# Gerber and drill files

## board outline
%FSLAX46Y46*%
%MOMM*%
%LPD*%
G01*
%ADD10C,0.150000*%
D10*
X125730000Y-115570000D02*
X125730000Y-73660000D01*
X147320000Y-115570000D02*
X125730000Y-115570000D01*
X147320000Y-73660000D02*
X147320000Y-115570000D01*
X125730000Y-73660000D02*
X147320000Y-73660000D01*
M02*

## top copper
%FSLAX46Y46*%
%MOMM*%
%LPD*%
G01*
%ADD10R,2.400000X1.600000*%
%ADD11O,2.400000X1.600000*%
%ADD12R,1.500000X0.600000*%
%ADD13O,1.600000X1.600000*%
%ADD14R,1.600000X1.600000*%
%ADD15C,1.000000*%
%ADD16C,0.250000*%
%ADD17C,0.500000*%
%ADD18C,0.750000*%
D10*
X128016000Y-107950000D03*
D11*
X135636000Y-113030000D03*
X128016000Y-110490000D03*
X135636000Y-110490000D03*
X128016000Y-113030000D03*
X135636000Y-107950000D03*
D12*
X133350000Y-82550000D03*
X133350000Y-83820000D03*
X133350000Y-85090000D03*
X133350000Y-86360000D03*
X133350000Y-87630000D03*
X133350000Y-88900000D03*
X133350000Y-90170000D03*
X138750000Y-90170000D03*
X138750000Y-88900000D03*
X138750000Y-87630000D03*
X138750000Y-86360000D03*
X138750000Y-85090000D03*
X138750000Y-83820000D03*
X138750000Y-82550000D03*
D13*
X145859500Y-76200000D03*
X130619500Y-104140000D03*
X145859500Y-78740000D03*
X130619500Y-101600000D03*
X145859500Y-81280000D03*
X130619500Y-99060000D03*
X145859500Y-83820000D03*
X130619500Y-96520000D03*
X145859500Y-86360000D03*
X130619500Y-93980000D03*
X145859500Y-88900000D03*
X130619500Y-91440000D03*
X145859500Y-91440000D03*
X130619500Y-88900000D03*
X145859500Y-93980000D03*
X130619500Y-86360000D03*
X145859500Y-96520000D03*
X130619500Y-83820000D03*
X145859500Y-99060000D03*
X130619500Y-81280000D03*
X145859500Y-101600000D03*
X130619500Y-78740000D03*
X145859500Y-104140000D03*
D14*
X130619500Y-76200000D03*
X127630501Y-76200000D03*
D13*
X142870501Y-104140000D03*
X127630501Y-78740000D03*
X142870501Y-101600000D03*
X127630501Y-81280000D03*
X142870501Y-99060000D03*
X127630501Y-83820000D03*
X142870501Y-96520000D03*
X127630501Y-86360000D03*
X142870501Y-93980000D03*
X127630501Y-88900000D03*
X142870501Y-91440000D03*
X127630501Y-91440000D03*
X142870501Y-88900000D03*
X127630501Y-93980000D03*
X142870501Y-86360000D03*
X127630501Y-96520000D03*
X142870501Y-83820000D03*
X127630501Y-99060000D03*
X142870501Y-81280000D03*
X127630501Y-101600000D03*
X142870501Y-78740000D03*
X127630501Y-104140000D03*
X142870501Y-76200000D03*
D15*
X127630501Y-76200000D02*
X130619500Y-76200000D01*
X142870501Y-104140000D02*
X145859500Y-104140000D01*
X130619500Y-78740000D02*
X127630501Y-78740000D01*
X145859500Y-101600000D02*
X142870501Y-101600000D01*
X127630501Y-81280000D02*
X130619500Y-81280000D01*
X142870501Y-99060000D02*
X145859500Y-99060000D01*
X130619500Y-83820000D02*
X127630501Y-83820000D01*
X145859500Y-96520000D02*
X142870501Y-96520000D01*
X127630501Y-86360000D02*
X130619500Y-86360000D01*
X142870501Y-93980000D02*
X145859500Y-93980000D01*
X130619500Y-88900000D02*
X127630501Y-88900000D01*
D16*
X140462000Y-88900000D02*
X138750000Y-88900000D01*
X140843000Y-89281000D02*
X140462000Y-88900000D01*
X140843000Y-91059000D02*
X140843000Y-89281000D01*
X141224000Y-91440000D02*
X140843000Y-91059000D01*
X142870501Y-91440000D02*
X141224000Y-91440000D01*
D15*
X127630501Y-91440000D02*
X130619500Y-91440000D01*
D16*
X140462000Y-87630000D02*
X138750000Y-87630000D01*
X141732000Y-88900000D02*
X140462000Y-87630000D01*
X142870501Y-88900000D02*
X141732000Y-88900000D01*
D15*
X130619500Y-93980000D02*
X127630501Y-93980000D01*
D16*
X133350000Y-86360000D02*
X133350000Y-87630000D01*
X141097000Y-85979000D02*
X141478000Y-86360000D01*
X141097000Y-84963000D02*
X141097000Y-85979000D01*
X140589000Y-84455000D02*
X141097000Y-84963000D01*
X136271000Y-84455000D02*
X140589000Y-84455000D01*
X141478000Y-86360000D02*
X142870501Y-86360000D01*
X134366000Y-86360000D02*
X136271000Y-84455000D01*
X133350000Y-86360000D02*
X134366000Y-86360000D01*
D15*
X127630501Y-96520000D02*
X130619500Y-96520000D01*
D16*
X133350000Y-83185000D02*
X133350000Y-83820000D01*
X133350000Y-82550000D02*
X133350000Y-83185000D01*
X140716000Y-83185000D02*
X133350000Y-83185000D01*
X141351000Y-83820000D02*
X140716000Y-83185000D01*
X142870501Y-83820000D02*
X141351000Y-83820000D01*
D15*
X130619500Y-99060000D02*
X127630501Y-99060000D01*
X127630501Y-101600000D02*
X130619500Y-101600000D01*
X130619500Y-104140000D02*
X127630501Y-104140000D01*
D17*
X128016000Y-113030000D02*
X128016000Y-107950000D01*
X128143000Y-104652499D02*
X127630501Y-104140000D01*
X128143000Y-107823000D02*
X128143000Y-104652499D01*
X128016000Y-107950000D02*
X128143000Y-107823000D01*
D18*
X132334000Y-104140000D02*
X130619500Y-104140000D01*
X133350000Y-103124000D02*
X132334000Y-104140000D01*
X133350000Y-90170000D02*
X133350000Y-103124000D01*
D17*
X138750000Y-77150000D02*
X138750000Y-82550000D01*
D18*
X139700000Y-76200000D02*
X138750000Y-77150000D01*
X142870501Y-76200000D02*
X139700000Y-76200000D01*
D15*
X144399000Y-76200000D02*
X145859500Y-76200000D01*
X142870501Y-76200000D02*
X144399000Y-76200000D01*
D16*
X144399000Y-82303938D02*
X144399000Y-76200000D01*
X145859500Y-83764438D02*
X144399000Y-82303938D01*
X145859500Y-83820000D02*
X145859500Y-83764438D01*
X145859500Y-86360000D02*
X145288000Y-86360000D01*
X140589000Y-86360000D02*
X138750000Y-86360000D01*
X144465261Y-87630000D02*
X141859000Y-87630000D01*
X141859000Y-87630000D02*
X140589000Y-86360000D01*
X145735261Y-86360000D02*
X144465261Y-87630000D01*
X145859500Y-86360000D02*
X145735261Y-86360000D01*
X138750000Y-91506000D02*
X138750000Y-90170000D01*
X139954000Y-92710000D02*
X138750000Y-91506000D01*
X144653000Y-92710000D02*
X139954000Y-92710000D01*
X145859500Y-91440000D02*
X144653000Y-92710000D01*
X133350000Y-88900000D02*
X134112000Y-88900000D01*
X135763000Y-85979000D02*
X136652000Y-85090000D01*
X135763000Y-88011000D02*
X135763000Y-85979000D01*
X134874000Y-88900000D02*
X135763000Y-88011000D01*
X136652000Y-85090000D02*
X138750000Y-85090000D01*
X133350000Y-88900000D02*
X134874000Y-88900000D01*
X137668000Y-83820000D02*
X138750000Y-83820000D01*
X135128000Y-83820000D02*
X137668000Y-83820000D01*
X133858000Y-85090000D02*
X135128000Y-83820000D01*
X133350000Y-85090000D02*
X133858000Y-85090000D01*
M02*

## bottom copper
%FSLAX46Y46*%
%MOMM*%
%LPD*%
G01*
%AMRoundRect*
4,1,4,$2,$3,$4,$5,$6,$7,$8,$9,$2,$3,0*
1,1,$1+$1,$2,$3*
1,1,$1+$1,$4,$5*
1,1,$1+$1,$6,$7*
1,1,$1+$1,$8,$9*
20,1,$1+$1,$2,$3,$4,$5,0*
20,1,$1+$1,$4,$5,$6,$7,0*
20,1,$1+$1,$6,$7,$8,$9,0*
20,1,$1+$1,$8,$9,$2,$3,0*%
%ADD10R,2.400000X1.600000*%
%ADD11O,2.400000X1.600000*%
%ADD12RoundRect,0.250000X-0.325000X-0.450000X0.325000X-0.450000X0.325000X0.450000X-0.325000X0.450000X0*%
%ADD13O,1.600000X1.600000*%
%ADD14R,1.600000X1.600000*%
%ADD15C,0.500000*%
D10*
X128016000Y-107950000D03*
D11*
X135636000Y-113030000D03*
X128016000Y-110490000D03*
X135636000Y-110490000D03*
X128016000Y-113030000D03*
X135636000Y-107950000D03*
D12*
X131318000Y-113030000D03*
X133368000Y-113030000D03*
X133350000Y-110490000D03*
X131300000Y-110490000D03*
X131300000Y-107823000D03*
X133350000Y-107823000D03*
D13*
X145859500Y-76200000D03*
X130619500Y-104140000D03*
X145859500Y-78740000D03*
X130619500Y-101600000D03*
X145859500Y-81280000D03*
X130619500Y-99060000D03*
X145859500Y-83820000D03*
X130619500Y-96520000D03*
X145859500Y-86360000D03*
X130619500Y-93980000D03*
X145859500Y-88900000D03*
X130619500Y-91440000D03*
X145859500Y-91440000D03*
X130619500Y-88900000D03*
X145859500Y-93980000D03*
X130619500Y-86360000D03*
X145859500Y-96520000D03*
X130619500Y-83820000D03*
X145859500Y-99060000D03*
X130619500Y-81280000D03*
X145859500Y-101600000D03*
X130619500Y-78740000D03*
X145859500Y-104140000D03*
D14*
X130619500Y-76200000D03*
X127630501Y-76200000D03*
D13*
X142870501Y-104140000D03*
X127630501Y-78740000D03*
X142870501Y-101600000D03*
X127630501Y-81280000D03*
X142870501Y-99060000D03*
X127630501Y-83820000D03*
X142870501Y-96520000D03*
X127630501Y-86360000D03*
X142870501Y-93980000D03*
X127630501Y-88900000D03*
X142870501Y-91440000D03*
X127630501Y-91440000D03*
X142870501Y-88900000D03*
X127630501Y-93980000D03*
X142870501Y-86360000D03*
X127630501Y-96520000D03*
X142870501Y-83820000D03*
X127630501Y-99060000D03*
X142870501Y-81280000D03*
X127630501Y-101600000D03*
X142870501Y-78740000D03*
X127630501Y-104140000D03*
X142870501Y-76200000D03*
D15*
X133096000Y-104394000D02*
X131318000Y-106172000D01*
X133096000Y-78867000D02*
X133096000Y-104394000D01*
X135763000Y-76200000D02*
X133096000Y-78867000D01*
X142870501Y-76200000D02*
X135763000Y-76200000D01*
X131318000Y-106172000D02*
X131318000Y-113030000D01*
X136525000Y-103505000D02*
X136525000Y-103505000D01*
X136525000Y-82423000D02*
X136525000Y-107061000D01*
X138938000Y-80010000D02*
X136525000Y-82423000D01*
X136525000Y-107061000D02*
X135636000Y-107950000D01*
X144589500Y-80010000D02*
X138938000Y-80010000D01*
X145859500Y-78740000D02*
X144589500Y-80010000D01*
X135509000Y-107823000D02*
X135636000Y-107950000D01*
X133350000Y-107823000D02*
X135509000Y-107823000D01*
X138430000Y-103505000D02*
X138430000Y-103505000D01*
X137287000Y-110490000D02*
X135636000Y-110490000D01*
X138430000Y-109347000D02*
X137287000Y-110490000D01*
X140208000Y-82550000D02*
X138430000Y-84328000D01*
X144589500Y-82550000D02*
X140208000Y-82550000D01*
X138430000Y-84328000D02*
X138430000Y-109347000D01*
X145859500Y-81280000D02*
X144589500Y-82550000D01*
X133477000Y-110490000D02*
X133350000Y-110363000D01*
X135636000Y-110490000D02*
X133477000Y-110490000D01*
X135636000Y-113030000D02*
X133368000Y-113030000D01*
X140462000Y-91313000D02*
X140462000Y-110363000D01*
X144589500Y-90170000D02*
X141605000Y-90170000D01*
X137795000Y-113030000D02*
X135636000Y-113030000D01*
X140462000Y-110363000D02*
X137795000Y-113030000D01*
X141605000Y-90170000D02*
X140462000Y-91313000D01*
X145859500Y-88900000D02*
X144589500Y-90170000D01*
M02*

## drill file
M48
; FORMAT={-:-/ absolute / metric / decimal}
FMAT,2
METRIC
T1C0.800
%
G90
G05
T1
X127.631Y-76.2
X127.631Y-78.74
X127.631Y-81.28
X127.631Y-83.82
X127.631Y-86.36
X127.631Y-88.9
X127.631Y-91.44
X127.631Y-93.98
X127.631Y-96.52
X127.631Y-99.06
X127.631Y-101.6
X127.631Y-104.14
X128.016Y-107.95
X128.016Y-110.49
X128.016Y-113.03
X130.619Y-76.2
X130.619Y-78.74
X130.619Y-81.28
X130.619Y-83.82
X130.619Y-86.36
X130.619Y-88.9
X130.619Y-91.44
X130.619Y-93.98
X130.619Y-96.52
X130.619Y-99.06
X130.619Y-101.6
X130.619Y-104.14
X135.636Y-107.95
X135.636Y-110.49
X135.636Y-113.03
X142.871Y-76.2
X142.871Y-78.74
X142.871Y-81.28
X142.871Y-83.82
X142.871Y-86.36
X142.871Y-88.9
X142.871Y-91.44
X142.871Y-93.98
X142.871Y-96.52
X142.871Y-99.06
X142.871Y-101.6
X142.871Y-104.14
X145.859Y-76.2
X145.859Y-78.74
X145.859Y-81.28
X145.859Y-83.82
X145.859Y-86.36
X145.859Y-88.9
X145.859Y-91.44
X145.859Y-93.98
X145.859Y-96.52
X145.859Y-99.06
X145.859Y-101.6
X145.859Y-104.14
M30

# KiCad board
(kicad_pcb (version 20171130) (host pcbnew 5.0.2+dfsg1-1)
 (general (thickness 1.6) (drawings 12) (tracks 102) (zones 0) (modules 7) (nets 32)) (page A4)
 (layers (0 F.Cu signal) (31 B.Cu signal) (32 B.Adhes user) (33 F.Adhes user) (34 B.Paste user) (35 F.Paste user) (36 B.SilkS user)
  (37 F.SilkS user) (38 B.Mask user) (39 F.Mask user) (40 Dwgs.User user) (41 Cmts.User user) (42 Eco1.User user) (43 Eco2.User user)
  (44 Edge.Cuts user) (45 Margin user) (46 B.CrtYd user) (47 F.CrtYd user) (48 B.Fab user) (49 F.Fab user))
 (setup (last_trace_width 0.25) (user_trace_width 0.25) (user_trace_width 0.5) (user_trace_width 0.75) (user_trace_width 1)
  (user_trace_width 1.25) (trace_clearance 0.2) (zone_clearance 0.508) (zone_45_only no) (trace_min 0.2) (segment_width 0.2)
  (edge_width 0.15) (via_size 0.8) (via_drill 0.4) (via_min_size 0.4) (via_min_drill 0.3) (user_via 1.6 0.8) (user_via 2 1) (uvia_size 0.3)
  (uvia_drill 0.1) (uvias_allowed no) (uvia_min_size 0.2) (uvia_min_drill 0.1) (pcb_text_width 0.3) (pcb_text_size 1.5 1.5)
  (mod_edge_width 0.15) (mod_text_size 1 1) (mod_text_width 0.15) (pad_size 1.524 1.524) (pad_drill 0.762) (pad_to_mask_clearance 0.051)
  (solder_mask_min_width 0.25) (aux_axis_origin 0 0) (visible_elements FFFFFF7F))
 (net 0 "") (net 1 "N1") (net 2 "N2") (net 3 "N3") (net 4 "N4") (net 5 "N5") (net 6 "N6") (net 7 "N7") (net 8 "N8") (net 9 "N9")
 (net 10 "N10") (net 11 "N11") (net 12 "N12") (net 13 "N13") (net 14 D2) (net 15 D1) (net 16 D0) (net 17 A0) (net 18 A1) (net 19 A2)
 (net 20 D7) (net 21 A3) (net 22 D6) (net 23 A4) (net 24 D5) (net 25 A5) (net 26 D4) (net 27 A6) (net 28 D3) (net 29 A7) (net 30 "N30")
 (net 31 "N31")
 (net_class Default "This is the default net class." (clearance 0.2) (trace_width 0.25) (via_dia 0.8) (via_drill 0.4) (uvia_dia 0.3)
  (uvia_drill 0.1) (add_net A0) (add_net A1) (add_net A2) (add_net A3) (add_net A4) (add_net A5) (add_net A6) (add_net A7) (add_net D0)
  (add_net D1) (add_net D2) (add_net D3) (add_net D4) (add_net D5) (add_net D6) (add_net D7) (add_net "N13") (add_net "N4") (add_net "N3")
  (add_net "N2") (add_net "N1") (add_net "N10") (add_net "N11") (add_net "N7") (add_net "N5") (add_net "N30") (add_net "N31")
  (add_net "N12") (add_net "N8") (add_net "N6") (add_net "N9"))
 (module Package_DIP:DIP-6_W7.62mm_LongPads (layer F.Cu) (at 128.016 107.95)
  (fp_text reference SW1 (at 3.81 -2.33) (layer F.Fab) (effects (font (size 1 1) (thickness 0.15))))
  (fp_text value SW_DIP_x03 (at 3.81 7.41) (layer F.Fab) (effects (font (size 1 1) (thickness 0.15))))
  (pad 1 thru_hole rect (at 0 0) (size 2.4 1.6) (drill 0.8) (layers *.Cu *.Mask) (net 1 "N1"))
  (pad 4 thru_hole oval (at 7.62 5.08) (size 2.4 1.6) (drill 0.8) (layers *.Cu *.Mask) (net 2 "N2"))
  (pad 2 thru_hole oval (at 0 2.54) (size 2.4 1.6) (drill 0.8) (layers *.Cu *.Mask) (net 1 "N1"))
  (pad 5 thru_hole oval (at 7.62 2.54) (size 2.4 1.6) (drill 0.8) (layers *.Cu *.Mask) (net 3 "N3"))
  (pad 3 thru_hole oval (at 0 5.08) (size 2.4 1.6) (drill 0.8) (layers *.Cu *.Mask) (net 1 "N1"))
  (pad 6 thru_hole oval (at 7.62 0) (size 2.4 1.6) (drill 0.8) (layers *.Cu *.Mask) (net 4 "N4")))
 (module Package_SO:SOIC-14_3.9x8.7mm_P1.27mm (layer F.Cu) (at 136.05 86.36)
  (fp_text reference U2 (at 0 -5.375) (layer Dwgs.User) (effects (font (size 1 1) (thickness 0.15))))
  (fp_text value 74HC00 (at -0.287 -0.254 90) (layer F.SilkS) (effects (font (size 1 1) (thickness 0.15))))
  (pad 1 smd rect (at -2.7 -3.81) (size 1.5 0.6) (layers F.Cu F.Paste F.Mask) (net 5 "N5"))
  (pad 2 smd rect (at -2.7 -2.54) (size 1.5 0.6) (layers F.Cu F.Paste F.Mask) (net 5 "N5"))
  (pad 3 smd rect (at -2.7 -1.27) (size 1.5 0.6) (layers F.Cu F.Paste F.Mask) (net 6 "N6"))
  (pad 4 smd rect (at -2.7 0) (size 1.5 0.6) (layers F.Cu F.Paste F.Mask) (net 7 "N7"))
  (pad 5 smd rect (at -2.7 1.27) (size 1.5 0.6) (layers F.Cu F.Paste F.Mask) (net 7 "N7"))
  (pad 6 smd rect (at -2.7 2.54) (size 1.5 0.6) (layers F.Cu F.Paste F.Mask) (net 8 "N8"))
  (pad 7 smd rect (at -2.7 3.81) (size 1.5 0.6) (layers F.Cu F.Paste F.Mask) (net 1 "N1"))
  (pad 8 smd rect (at 2.7 3.81) (size 1.5 0.6) (layers F.Cu F.Paste F.Mask) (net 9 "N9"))
  (pad 9 smd rect (at 2.7 2.54) (size 1.5 0.6) (layers F.Cu F.Paste F.Mask) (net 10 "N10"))
  (pad 10 smd rect (at 2.7 1.27) (size 1.5 0.6) (layers F.Cu F.Paste F.Mask) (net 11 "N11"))
  (pad 11 smd rect (at 2.7 0) (size 1.5 0.6) (layers F.Cu F.Paste F.Mask) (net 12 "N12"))
  (pad 12 smd rect (at 2.7 -1.27) (size 1.5 0.6) (layers F.Cu F.Paste F.Mask) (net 8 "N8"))
  (pad 13 smd rect (at 2.7 -2.54) (size 1.5 0.6) (layers F.Cu F.Paste F.Mask) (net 6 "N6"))
  (pad 14 smd rect (at 2.7 -3.81) (size 1.5 0.6) (layers F.Cu F.Paste F.Mask) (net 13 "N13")))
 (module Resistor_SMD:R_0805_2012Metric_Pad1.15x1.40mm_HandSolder (layer B.Cu) (at 132.343 113.03)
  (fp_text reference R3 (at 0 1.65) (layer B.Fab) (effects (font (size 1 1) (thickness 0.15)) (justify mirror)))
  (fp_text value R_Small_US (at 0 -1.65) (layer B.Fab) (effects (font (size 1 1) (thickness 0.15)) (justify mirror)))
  (pad 1 smd roundrect (at -1.025 0) (size 1.15 1.4) (layers B.Cu B.Paste B.Mask) (roundrect_rratio 0.217391) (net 13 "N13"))
  (pad 2 smd roundrect (at 1.025 0) (size 1.15 1.4) (layers B.Cu B.Paste B.Mask) (roundrect_rratio 0.217391) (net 2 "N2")))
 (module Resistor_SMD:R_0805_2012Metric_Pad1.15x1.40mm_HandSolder (layer B.Cu) (at 132.325 110.49)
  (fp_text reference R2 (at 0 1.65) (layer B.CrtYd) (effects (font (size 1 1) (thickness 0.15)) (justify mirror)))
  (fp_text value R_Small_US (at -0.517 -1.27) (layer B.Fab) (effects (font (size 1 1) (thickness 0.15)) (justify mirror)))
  (pad 2 smd roundrect (at 1.025 0) (size 1.15 1.4) (layers B.Cu B.Paste B.Mask) (roundrect_rratio 0.217391) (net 3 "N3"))
  (pad 1 smd roundrect (at -1.025 0) (size 1.15 1.4) (layers B.Cu B.Paste B.Mask) (roundrect_rratio 0.217391) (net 13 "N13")))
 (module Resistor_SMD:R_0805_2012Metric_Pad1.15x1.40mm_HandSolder (layer B.Cu) (at 132.325 107.823)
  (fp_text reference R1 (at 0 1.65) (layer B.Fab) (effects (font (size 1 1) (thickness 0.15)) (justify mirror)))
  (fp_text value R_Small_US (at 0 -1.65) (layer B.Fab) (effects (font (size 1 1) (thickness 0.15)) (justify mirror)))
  (pad 1 smd roundrect (at -1.025 0) (size 1.15 1.4) (layers B.Cu B.Paste B.Mask) (roundrect_rratio 0.217391) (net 13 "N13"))
  (pad 2 smd roundrect (at 1.025 0) (size 1.15 1.4) (layers B.Cu B.Paste B.Mask) (roundrect_rratio 0.217391) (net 4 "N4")))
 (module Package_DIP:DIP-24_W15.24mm (layer F.Cu) (at 130.6195 76.2)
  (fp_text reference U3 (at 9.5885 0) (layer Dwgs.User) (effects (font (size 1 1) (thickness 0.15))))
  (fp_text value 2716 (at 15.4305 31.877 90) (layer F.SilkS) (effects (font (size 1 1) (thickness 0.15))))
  (pad 24 thru_hole oval (at 15.24 0) (size 1.6 1.6) (drill 0.8) (layers *.Cu *.Mask) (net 13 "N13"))
  (pad 12 thru_hole oval (at 0 27.94) (size 1.6 1.6) (drill 0.8) (layers *.Cu *.Mask) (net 1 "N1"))
  (pad 23 thru_hole oval (at 15.24 2.54) (size 1.6 1.6) (drill 0.8) (layers *.Cu *.Mask) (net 4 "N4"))
  (pad 11 thru_hole oval (at 0 25.4) (size 1.6 1.6) (drill 0.8) (layers *.Cu *.Mask) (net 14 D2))
  (pad 22 thru_hole oval (at 15.24 5.08) (size 1.6 1.6) (drill 0.8) (layers *.Cu *.Mask) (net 3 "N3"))
  (pad 10 thru_hole oval (at 0 22.86) (size 1.6 1.6) (drill 0.8) (layers *.Cu *.Mask) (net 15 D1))
  (pad 21 thru_hole oval (at 15.24 7.62) (size 1.6 1.6) (drill 0.8) (layers *.Cu *.Mask) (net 13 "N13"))
  (pad 9 thru_hole oval (at 0 20.32) (size 1.6 1.6) (drill 0.8) (layers *.Cu *.Mask) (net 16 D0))
  (pad 20 thru_hole oval (at 15.24 10.16) (size 1.6 1.6) (drill 0.8) (layers *.Cu *.Mask) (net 12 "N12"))
  (pad 8 thru_hole oval (at 0 17.78) (size 1.6 1.6) (drill 0.8) (layers *.Cu *.Mask) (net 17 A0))
  (pad 19 thru_hole oval (at 15.24 12.7) (size 1.6 1.6) (drill 0.8) (layers *.Cu *.Mask) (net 2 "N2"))
  (pad 7 thru_hole oval (at 0 15.24) (size 1.6 1.6) (drill 0.8) (layers *.Cu *.Mask) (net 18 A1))
  (pad 18 thru_hole oval (at 15.24 15.24) (size 1.6 1.6) (drill 0.8) (layers *.Cu *.Mask) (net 9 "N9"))
  (pad 6 thru_hole oval (at 0 12.7) (size 1.6 1.6) (drill 0.8) (layers *.Cu *.Mask) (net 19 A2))
  (pad 17 thru_hole oval (at 15.24 17.78) (size 1.6 1.6) (drill 0.8) (layers *.Cu *.Mask) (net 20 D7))
  (pad 5 thru_hole oval (at 0 10.16) (size 1.6 1.6) (drill 0.8) (layers *.Cu *.Mask) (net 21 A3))
  (pad 16 thru_hole oval (at 15.24 20.32) (size 1.6 1.6) (drill 0.8) (layers *.Cu *.Mask) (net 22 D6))
  (pad 4 thru_hole oval (at 0 7.62) (size 1.6 1.6) (drill 0.8) (layers *.Cu *.Mask) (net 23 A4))
  (pad 15 thru_hole oval (at 15.24 22.86) (size 1.6 1.6) (drill 0.8) (layers *.Cu *.Mask) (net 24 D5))
  (pad 3 thru_hole oval (at 0 5.08) (size 1.6 1.6) (drill 0.8) (layers *.Cu *.Mask) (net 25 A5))
  (pad 14 thru_hole oval (at 15.24 25.4) (size 1.6 1.6) (drill 0.8) (layers *.Cu *.Mask) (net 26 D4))
  (pad 2 thru_hole oval (at 0 2.54) (size 1.6 1.6) (drill 0.8) (layers *.Cu *.Mask) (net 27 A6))
  (pad 13 thru_hole oval (at 15.24 27.94) (size 1.6 1.6) (drill 0.8) (layers *.Cu *.Mask) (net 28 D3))
  (pad 1 thru_hole rect (at 0 0) (size 1.6 1.6) (drill 0.8) (layers *.Cu *.Mask) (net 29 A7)))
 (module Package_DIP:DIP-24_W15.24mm (layer F.Cu) (at 127.630501 76.2)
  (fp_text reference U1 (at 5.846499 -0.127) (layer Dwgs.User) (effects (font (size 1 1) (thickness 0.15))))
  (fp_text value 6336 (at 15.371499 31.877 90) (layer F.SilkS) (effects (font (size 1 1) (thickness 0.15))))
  (pad 1 thru_hole rect (at 0 0) (size 1.6 1.6) (drill 0.8) (layers *.Cu *.Mask) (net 29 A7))
  (pad 13 thru_hole oval (at 15.24 27.94) (size 1.6 1.6) (drill 0.8) (layers *.Cu *.Mask) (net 28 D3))
  (pad 2 thru_hole oval (at 0 2.54) (size 1.6 1.6) (drill 0.8) (layers *.Cu *.Mask) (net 27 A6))
  (pad 14 thru_hole oval (at 15.24 25.4) (size 1.6 1.6) (drill 0.8) (layers *.Cu *.Mask) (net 26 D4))
  (pad 3 thru_hole oval (at 0 5.08) (size 1.6 1.6) (drill 0.8) (layers *.Cu *.Mask) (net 25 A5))
  (pad 15 thru_hole oval (at 15.24 22.86) (size 1.6 1.6) (drill 0.8) (layers *.Cu *.Mask) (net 24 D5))
  (pad 4 thru_hole oval (at 0 7.62) (size 1.6 1.6) (drill 0.8) (layers *.Cu *.Mask) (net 23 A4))
  (pad 16 thru_hole oval (at 15.24 20.32) (size 1.6 1.6) (drill 0.8) (layers *.Cu *.Mask) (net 22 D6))
  (pad 5 thru_hole oval (at 0 10.16) (size 1.6 1.6) (drill 0.8) (layers *.Cu *.Mask) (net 21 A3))
  (pad 17 thru_hole oval (at 15.24 17.78) (size 1.6 1.6) (drill 0.8) (layers *.Cu *.Mask) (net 20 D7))
  (pad 6 thru_hole oval (at 0 12.7) (size 1.6 1.6) (drill 0.8) (layers *.Cu *.Mask) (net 19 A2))
  (pad 18 thru_hole oval (at 15.24 15.24) (size 1.6 1.6) (drill 0.8) (layers *.Cu *.Mask) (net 10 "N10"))
  (pad 7 thru_hole oval (at 0 15.24) (size 1.6 1.6) (drill 0.8) (layers *.Cu *.Mask) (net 18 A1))
  (pad 19 thru_hole oval (at 15.24 12.7) (size 1.6 1.6) (drill 0.8) (layers *.Cu *.Mask) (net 11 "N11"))
  (pad 8 thru_hole oval (at 0 17.78) (size 1.6 1.6) (drill 0.8) (layers *.Cu *.Mask) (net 17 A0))
  (pad 20 thru_hole oval (at 15.24 10.16) (size 1.6 1.6) (drill 0.8) (layers *.Cu *.Mask) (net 7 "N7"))
  (pad 9 thru_hole oval (at 0 20.32) (size 1.6 1.6) (drill 0.8) (layers *.Cu *.Mask) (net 16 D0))
  (pad 21 thru_hole oval (at 15.24 7.62) (size 1.6 1.6) (drill 0.8) (layers *.Cu *.Mask) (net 5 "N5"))
  (pad 10 thru_hole oval (at 0 22.86) (size 1.6 1.6) (drill 0.8) (layers *.Cu *.Mask) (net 15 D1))
  (pad 22 thru_hole oval (at 15.24 5.08) (size 1.6 1.6) (drill 0.8) (layers *.Cu *.Mask) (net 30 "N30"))
  (pad 11 thru_hole oval (at 0 25.4) (size 1.6 1.6) (drill 0.8) (layers *.Cu *.Mask) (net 14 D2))
  (pad 23 thru_hole oval (at 15.24 2.54) (size 1.6 1.6) (drill 0.8) (layers *.Cu *.Mask) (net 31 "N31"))
  (pad 12 thru_hole oval (at 0 27.94) (size 1.6 1.6) (drill 0.8) (layers *.Cu *.Mask) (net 1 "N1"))
  (pad 24 thru_hole oval (at 15.24 0) (size 1.6 1.6) (drill 0.8) (layers *.Cu *.Mask) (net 13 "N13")))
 (gr_line (start 125.73 115.57) (end 125.73 73.66) (layer Edge.Cuts) (width 0.15))
 (gr_line (start 147.32 115.57) (end 125.73 115.57) (layer Edge.Cuts) (width 0.15))
 (gr_line (start 147.32 73.66) (end 147.32 115.57) (layer Edge.Cuts) (width 0.15))
 (gr_line (start 125.73 73.66) (end 147.32 73.66) (layer Edge.Cuts) (width 0.15))
 (segment (start 127.630501 76.2) (end 130.6195 76.2) (width 1) (layer F.Cu) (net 29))
 (segment (start 142.870501 104.14) (end 145.8595 104.14) (width 1) (layer F.Cu) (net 28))
 (segment (start 130.6195 78.74) (end 127.630501 78.74) (width 1) (layer F.Cu) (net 27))
 (segment (start 145.8595 101.6) (end 142.870501 101.6) (width 1) (layer F.Cu) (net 26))
 (segment (start 127.630501 81.28) (end 130.6195 81.28) (width 1) (layer F.Cu) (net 25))
 (segment (start 142.870501 99.06) (end 145.8595 99.06) (width 1) (layer F.Cu) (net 24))
 (segment (start 130.6195 83.82) (end 127.630501 83.82) (width 1) (layer F.Cu) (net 23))
 (segment (start 145.8595 96.52) (end 142.870501 96.52) (width 1) (layer F.Cu) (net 22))
 (segment (start 127.630501 86.36) (end 130.6195 86.36) (width 1) (layer F.Cu) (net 21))
 (segment (start 142.870501 93.98) (end 145.8595 93.98) (width 1) (layer F.Cu) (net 20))
 (segment (start 130.6195 88.9) (end 127.630501 88.9) (width 1) (layer F.Cu) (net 19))
 (segment (start 140.462 88.9) (end 138.75 88.9) (width 0.25) (layer F.Cu) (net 10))
 (segment (start 140.843 89.281) (end 140.462 88.9) (width 0.25) (layer F.Cu) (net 10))
 (segment (start 140.843 91.059) (end 140.843 89.281) (width 0.25) (layer F.Cu) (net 10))
 (segment (start 141.224 91.44) (end 140.843 91.059) (width 0.25) (layer F.Cu) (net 10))
 (segment (start 142.870501 91.44) (end 141.224 91.44) (width 0.25) (layer F.Cu) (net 10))
 (segment (start 127.630501 91.44) (end 130.6195 91.44) (width 1) (layer F.Cu) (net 18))
 (segment (start 140.462 87.63) (end 138.75 87.63) (width 0.25) (layer F.Cu) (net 11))
 (segment (start 141.732 88.9) (end 140.462 87.63) (width 0.25) (layer F.Cu) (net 11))
 (segment (start 142.870501 88.9) (end 141.732 88.9) (width 0.25) (layer F.Cu) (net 11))
 (segment (start 130.6195 93.98) (end 127.630501 93.98) (width 1) (layer F.Cu) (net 17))
 (segment (start 133.35 86.36) (end 133.35 87.63) (width 0.25) (layer F.Cu) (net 7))
 (segment (start 141.097 85.979) (end 141.478 86.36) (width 0.25) (layer F.Cu) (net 7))
 (segment (start 141.097 84.963) (end 141.097 85.979) (width 0.25) (layer F.Cu) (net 7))
 (segment (start 140.589 84.455) (end 141.097 84.963) (width 0.25) (layer F.Cu) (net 7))
 (segment (start 136.271 84.455) (end 140.589 84.455) (width 0.25) (layer F.Cu) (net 7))
 (segment (start 141.478 86.36) (end 142.870501 86.36) (width 0.25) (layer F.Cu) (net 7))
 (segment (start 134.366 86.36) (end 136.271 84.455) (width 0.25) (layer F.Cu) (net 7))
 (segment (start 133.35 86.36) (end 134.366 86.36) (width 0.25) (layer F.Cu) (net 7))
 (segment (start 127.630501 96.52) (end 130.6195 96.52) (width 1) (layer F.Cu) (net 16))
 (segment (start 133.35 83.185) (end 133.35 83.82) (width 0.25) (layer F.Cu) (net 5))
 (segment (start 133.35 82.55) (end 133.35 83.185) (width 0.25) (layer F.Cu) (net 5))
 (segment (start 140.716 83.185) (end 133.35 83.185) (width 0.25) (layer F.Cu) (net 5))
 (segment (start 141.351 83.82) (end 140.716 83.185) (width 0.25) (layer F.Cu) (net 5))
 (segment (start 142.870501 83.82) (end 141.351 83.82) (width 0.25) (layer F.Cu) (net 5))
 (segment (start 130.6195 99.06) (end 127.630501 99.06) (width 1) (layer F.Cu) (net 15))
 (segment (start 127.630501 101.6) (end 130.6195 101.6) (width 1) (layer F.Cu) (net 14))
 (segment (start 130.6195 104.14) (end 127.630501 104.14) (width 1) (layer F.Cu) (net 1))
 (segment (start 128.016 113.03) (end 128.016 107.95) (width 0.5) (layer F.Cu) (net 1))
 (segment (start 128.143 104.652499) (end 127.630501 104.14) (width 0.5) (layer F.Cu) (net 1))
 (segment (start 128.143 107.823) (end 128.143 104.652499) (width 0.5) (layer F.Cu) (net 1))
 (segment (start 128.016 107.95) (end 128.143 107.823) (width 0.5) (layer F.Cu) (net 1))
 (segment (start 132.334 104.14) (end 130.6195 104.14) (width 0.75) (layer F.Cu) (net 1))
 (segment (start 133.35 103.124) (end 132.334 104.14) (width 0.75) (layer F.Cu) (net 1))
 (segment (start 133.35 90.17) (end 133.35 103.124) (width 0.75) (layer F.Cu) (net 1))
 (segment (start 138.75 77.15) (end 138.75 82.55) (width 0.5) (layer F.Cu) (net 13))
 (segment (start 139.7 76.2) (end 138.75 77.15) (width 0.75) (layer F.Cu) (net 13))
 (segment (start 142.870501 76.2) (end 139.7 76.2) (width 0.75) (layer F.Cu) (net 13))
 (segment (start 144.399 76.2) (end 145.8595 76.2) (width 1) (layer F.Cu) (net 13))
 (segment (start 142.870501 76.2) (end 144.399 76.2) (width 1) (layer F.Cu) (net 13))
 (segment (start 144.399 82.303938) (end 144.399 76.2) (width 0.25) (layer F.Cu) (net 13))
 (segment (start 145.8595 83.764438) (end 144.399 82.303938) (width 0.25) (layer F.Cu) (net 13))
 (segment (start 145.8595 83.82) (end 145.8595 83.764438) (width 0.25) (layer F.Cu) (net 13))
 (segment (start 133.096 104.394) (end 131.318 106.172) (width 0.5) (layer B.Cu) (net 13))
 (segment (start 133.096 78.867) (end 133.096 104.394) (width 0.5) (layer B.Cu) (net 13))
 (segment (start 135.763 76.2) (end 133.096 78.867) (width 0.5) (layer B.Cu) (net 13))
 (segment (start 142.870501 76.2) (end 135.763 76.2) (width 0.5) (layer B.Cu) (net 13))
 (segment (start 131.318 106.172) (end 131.318 113.03) (width 0.5) (layer B.Cu) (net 13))
 (segment (start 136.525 103.505) (end 136.525 103.505) (width 0.5) (layer B.Cu) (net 4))
 (segment (start 136.525 82.423) (end 136.525 107.061) (width 0.5) (layer B.Cu) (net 4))
 (segment (start 138.938 80.01) (end 136.525 82.423) (width 0.5) (layer B.Cu) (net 4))
 (segment (start 136.525 107.061) (end 135.636 107.95) (width 0.5) (layer B.Cu) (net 4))
 (segment (start 144.5895 80.01) (end 138.938 80.01) (width 0.5) (layer B.Cu) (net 4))
 (segment (start 145.8595 78.74) (end 144.5895 80.01) (width 0.5) (layer B.Cu) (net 4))
 (segment (start 135.509 107.823) (end 135.636 107.95) (width 0.5) (layer B.Cu) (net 4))
 (segment (start 133.35 107.823) (end 135.509 107.823) (width 0.5) (layer B.Cu) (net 4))
 (segment (start 138.43 103.505) (end 138.43 103.505) (width 0.5) (layer B.Cu) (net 3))
 (segment (start 137.287 110.49) (end 135.636 110.49) (width 0.5) (layer B.Cu) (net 3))
 (segment (start 138.43 109.347) (end 137.287 110.49) (width 0.5) (layer B.Cu) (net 3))
 (segment (start 140.208 82.55) (end 138.43 84.328) (width 0.5) (layer B.Cu) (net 3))
 (segment (start 144.5895 82.55) (end 140.208 82.55) (width 0.5) (layer B.Cu) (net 3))
 (segment (start 138.43 84.328) (end 138.43 109.347) (width 0.5) (layer B.Cu) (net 3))
 (segment (start 145.8595 81.28) (end 144.5895 82.55) (width 0.5) (layer B.Cu) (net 3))
 (segment (start 133.477 110.49) (end 133.35 110.363) (width 0.5) (layer B.Cu) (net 3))
 (segment (start 135.636 110.49) (end 133.477 110.49) (width 0.5) (layer B.Cu) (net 3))
 (segment (start 145.8595 86.36) (end 145.288 86.36) (width 0.25) (layer F.Cu) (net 12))
 (segment (start 140.589 86.36) (end 138.75 86.36) (width 0.25) (layer F.Cu) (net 12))
 (segment (start 144.465261 87.63) (end 141.859 87.63) (width 0.25) (layer F.Cu) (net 12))
 (segment (start 141.859 87.63) (end 140.589 86.36) (width 0.25) (layer F.Cu) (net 12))
 (segment (start 145.735261 86.36) (end 144.465261 87.63) (width 0.25) (layer F.Cu) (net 12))
 (segment (start 145.8595 86.36) (end 145.735261 86.36) (width 0.25) (layer F.Cu) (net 12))
 (segment (start 135.636 113.03) (end 133.368 113.03) (width 0.5) (layer B.Cu) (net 2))
 (segment (start 140.462 91.313) (end 140.462 110.363) (width 0.5) (layer B.Cu) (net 2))
 (segment (start 144.5895 90.17) (end 141.605 90.17) (width 0.5) (layer B.Cu) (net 2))
 (segment (start 137.795 113.03) (end 135.636 113.03) (width 0.5) (layer B.Cu) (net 2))
 (segment (start 140.462 110.363) (end 137.795 113.03) (width 0.5) (layer B.Cu) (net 2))
 (segment (start 141.605 90.17) (end 140.462 91.313) (width 0.5) (layer B.Cu) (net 2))
 (segment (start 145.8595 88.9) (end 144.5895 90.17) (width 0.5) (layer B.Cu) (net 2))
 (segment (start 138.75 91.506) (end 138.75 90.17) (width 0.25) (layer F.Cu) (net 9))
 (segment (start 139.954 92.71) (end 138.75 91.506) (width 0.25) (layer F.Cu) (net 9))
 (segment (start 144.653 92.71) (end 139.954 92.71) (width 0.25) (layer F.Cu) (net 9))
 (segment (start 145.8595 91.44) (end 144.653 92.71) (width 0.25) (layer F.Cu) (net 9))
 (segment (start 133.35 88.9) (end 134.112 88.9) (width 0.25) (layer F.Cu) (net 8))
 (segment (start 135.763 85.979) (end 136.652 85.09) (width 0.25) (layer F.Cu) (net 8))
 (segment (start 135.763 88.011) (end 135.763 85.979) (width 0.25) (layer F.Cu) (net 8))
 (segment (start 134.874 88.9) (end 135.763 88.011) (width 0.25) (layer F.Cu) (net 8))
 (segment (start 136.652 85.09) (end 138.75 85.09) (width 0.25) (layer F.Cu) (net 8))
 (segment (start 133.35 88.9) (end 134.874 88.9) (width 0.25) (layer F.Cu) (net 8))
 (segment (start 137.668 83.82) (end 138.75 83.82) (width 0.25) (layer F.Cu) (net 6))
 (segment (start 135.128 83.82) (end 137.668 83.82) (width 0.25) (layer F.Cu) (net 6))
 (segment (start 133.858 85.09) (end 135.128 83.82) (width 0.25) (layer F.Cu) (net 6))
 (segment (start 133.35 85.09) (end 133.858 85.09) (width 0.25) (layer F.Cu) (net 6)))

